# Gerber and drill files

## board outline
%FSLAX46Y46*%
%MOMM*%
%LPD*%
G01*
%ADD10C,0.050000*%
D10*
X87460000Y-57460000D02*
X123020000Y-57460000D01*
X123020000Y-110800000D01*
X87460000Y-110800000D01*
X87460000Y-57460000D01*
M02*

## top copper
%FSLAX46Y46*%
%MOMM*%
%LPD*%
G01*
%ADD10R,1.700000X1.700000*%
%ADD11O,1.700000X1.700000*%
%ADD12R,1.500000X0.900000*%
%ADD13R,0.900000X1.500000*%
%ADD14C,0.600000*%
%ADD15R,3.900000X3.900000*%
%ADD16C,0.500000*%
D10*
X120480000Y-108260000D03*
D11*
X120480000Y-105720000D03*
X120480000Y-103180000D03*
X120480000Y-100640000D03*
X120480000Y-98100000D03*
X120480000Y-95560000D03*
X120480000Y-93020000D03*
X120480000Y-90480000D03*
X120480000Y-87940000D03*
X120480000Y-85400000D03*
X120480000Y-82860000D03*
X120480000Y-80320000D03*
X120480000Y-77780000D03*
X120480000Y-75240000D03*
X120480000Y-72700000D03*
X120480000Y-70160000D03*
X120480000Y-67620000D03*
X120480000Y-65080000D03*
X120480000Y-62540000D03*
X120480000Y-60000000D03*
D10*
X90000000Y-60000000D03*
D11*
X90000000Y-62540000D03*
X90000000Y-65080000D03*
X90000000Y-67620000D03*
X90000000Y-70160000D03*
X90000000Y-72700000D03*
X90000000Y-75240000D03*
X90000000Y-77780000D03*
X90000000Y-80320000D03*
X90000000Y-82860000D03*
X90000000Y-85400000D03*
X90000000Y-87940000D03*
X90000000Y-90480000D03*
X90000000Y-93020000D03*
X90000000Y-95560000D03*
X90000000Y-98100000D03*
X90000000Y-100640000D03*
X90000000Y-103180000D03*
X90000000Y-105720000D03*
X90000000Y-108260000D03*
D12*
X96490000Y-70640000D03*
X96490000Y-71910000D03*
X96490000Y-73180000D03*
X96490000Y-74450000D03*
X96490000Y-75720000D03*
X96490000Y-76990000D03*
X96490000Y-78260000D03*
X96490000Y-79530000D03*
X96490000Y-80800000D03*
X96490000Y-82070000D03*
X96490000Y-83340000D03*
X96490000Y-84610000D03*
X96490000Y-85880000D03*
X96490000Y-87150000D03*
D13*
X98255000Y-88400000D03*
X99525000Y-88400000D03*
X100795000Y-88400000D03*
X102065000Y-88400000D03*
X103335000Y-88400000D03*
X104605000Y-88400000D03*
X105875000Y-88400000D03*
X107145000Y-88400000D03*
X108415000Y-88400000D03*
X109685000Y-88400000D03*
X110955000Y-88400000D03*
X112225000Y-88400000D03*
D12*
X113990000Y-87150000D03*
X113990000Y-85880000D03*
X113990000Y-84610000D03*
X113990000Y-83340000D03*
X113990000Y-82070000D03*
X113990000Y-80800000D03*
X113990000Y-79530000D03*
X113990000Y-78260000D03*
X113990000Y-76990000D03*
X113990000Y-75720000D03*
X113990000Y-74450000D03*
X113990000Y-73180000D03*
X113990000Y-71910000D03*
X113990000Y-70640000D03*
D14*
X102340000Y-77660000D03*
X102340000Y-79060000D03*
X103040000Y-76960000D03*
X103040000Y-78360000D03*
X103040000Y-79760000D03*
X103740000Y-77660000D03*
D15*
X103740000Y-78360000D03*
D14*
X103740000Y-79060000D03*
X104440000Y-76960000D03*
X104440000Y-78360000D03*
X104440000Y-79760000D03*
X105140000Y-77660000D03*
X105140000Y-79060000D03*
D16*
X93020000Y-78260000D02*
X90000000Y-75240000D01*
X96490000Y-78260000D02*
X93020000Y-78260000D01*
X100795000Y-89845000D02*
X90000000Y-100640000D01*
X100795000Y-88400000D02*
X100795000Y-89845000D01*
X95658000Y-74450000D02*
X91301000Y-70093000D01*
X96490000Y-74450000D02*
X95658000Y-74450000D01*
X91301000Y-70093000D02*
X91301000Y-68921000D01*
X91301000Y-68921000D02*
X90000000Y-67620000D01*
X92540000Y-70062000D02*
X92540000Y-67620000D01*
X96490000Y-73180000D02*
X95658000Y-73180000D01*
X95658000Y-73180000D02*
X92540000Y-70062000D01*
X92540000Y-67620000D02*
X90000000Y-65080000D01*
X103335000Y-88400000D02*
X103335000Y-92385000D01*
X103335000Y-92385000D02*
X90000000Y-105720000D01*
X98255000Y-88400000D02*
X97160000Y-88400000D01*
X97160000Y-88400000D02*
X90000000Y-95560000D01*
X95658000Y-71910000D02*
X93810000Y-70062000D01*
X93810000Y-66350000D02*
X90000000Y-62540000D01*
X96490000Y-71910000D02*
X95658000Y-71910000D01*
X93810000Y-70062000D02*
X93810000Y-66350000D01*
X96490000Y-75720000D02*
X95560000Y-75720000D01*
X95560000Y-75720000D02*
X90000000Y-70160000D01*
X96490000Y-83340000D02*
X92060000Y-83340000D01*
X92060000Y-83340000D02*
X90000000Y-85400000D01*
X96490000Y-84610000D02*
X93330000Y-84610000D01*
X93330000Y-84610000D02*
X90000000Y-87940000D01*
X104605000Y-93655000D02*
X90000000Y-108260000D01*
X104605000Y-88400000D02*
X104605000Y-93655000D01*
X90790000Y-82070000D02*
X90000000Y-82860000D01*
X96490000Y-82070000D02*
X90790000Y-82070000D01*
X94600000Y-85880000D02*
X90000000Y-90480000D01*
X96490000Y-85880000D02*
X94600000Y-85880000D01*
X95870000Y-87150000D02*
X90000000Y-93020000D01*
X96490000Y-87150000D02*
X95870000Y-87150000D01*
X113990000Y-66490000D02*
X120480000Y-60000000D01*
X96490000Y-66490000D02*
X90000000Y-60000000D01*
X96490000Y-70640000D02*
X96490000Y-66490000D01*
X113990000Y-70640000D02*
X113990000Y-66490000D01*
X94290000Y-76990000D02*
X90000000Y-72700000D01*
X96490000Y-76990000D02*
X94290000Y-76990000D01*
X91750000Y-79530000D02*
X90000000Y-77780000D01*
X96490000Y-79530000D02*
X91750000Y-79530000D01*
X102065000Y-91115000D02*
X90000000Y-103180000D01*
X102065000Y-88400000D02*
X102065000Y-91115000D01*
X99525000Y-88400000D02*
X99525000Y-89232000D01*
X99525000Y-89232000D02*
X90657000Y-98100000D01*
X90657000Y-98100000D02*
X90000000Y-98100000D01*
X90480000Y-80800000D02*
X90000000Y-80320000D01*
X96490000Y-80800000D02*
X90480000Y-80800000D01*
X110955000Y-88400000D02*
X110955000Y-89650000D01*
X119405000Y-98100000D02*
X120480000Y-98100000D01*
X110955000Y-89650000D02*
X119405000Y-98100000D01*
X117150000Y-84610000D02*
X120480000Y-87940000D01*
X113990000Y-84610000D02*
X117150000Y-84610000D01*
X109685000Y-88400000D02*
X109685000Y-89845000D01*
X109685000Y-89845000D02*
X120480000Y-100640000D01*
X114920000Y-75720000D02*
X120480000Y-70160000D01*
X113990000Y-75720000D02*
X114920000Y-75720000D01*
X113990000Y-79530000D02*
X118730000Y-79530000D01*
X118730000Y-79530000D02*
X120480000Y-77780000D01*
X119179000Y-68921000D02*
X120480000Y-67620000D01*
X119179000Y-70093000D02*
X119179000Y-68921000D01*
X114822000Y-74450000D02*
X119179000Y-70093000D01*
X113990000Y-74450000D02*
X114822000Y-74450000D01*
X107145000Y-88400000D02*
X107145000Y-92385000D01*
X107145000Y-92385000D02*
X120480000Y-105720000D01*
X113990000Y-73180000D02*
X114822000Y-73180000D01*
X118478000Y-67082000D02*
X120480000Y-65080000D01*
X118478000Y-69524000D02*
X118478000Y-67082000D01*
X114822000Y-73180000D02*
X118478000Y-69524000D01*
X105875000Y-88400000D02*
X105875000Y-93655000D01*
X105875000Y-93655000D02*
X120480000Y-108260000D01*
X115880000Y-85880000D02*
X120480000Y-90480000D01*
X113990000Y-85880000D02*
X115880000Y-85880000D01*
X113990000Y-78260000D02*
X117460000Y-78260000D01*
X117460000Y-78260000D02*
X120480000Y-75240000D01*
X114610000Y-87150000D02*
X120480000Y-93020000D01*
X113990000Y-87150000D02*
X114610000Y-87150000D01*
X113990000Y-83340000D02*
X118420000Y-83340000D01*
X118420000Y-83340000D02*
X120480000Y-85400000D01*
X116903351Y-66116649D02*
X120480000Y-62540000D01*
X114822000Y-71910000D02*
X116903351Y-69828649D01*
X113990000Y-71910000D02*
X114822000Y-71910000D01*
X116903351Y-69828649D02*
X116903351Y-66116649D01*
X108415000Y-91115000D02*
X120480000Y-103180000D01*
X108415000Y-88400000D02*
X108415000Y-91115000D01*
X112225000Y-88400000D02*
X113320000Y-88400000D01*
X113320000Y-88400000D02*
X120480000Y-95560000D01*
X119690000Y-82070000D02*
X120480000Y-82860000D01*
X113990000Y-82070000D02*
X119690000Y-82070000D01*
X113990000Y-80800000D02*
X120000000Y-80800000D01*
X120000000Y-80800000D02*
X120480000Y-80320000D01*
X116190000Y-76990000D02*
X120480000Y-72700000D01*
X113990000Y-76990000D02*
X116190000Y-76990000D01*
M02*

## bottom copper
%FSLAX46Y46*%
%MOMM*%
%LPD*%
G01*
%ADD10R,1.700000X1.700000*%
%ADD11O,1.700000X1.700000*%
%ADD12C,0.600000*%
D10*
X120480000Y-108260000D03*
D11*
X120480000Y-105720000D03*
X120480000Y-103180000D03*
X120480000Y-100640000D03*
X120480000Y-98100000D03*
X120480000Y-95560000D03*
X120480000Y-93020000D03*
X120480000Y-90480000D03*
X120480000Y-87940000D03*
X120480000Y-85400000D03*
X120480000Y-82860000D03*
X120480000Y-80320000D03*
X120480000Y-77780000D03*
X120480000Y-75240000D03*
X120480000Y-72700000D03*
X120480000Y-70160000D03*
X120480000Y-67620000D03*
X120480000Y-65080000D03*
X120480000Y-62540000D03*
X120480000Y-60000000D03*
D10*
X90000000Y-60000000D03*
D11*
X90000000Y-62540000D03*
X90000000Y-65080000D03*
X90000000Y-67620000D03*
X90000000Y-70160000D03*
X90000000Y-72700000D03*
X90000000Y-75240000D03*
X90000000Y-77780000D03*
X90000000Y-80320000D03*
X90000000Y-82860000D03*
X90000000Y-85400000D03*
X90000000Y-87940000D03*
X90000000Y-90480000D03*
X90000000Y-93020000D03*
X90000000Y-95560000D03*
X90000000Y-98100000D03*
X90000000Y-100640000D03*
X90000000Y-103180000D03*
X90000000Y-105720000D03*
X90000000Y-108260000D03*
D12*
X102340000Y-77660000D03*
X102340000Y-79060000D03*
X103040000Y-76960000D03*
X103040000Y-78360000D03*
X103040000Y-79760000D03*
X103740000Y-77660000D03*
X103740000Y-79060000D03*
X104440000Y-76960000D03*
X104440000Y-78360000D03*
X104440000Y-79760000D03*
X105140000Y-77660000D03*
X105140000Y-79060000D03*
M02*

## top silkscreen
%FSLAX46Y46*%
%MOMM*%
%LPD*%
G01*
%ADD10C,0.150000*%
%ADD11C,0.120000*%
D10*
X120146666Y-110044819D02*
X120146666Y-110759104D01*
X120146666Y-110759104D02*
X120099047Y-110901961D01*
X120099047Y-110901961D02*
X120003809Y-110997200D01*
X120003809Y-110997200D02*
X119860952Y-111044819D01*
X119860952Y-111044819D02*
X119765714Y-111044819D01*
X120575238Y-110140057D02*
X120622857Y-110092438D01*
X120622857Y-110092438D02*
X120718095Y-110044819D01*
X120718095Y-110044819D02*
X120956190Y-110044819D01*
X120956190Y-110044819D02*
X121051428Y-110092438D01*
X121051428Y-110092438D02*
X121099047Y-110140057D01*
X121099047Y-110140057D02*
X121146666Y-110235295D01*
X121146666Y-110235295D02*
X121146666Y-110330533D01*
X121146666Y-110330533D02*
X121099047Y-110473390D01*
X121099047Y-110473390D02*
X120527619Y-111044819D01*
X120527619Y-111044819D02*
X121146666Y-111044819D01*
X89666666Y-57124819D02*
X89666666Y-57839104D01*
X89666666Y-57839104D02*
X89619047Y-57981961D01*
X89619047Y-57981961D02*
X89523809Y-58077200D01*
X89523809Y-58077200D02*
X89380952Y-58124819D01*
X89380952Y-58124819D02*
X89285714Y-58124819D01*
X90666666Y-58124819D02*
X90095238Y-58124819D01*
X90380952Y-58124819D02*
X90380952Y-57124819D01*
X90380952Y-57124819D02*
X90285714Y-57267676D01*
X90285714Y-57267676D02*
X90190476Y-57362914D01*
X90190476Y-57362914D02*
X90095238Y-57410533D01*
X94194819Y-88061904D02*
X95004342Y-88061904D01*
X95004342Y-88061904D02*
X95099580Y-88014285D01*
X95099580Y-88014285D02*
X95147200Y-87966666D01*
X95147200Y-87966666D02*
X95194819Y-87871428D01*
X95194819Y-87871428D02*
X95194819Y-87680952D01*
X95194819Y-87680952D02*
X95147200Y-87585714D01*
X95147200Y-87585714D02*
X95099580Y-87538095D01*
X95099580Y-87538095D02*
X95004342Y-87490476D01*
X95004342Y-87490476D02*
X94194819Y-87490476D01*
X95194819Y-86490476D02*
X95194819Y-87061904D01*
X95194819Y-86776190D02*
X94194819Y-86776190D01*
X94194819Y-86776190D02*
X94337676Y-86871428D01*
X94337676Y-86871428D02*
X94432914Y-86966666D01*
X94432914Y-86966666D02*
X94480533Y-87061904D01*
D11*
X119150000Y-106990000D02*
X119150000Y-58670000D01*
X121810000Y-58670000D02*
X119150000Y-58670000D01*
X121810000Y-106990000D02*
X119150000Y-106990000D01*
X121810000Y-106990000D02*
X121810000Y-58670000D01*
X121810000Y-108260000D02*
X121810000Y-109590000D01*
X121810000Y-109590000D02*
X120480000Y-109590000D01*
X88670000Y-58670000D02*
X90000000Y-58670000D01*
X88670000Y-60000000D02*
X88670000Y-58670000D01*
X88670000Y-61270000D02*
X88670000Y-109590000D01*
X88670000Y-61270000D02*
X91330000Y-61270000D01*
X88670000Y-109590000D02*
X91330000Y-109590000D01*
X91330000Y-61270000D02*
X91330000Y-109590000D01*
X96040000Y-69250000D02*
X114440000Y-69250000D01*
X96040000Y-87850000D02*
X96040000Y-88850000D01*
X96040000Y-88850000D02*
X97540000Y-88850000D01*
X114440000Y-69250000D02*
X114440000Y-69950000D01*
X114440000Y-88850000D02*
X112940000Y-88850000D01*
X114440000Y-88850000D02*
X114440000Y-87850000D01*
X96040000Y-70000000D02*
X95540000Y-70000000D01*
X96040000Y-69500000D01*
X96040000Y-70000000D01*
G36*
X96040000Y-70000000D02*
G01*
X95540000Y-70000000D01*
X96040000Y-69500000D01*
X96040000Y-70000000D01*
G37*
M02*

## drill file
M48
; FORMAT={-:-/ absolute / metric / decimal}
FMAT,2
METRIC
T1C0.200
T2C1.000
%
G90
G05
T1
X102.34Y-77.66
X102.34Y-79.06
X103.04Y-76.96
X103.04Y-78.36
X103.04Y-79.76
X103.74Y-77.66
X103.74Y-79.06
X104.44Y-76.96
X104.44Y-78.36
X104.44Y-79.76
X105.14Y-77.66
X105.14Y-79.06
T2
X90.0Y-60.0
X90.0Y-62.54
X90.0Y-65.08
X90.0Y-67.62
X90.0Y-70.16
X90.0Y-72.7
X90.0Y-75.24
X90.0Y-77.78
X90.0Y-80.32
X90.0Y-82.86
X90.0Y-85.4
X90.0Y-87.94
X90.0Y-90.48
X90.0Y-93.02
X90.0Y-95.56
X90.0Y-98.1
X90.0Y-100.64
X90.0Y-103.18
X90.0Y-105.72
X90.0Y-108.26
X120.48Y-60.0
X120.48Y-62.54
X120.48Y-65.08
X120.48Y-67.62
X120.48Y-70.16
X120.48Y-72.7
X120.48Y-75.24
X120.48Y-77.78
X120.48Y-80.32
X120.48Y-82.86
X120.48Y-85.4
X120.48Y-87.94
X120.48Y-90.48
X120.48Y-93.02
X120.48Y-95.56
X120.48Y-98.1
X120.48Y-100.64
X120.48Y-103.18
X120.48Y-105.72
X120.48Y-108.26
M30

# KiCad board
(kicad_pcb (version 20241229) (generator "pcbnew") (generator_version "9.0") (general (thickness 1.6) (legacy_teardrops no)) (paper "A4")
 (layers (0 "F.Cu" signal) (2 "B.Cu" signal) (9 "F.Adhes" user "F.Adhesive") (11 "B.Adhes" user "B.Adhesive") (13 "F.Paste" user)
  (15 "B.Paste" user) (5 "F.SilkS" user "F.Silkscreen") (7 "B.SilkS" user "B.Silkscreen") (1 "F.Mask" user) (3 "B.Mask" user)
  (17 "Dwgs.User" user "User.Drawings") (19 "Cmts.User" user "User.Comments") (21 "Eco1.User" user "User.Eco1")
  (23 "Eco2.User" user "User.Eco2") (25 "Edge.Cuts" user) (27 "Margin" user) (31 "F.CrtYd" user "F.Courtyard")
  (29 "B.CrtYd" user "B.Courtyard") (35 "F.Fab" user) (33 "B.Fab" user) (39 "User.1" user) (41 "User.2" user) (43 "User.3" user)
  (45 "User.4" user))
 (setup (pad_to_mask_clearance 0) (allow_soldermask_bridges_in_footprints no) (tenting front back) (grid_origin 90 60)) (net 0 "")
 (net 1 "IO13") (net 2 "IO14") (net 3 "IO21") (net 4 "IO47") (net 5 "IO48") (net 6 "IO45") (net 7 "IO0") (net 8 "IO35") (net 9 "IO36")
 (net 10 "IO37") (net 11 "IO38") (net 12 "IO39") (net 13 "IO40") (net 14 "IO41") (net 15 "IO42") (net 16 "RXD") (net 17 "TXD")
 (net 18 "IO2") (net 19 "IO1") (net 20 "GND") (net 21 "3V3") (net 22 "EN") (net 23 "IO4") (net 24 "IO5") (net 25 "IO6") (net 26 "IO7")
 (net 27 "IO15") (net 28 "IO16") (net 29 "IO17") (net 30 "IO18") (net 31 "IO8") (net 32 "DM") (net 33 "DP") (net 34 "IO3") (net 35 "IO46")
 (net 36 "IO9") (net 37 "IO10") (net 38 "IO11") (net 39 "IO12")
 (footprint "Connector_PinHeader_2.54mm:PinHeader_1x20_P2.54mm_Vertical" (layer "F.Cu") (at 120.48 108.26 180)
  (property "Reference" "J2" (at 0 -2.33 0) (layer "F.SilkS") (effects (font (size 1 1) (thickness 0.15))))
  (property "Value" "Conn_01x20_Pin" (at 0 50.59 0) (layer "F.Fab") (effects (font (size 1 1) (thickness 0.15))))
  (fp_line (start 1.33 1.27) (end 1.33 49.59) (stroke (width 0.12) (type solid)) (layer "F.SilkS"))
  (fp_line (start -1.33 49.59) (end 1.33 49.59) (stroke (width 0.12) (type solid)) (layer "F.SilkS"))
  (fp_line (start -1.33 1.27) (end 1.33 1.27) (stroke (width 0.12) (type solid)) (layer "F.SilkS"))
  (fp_line (start -1.33 1.27) (end -1.33 49.59) (stroke (width 0.12) (type solid)) (layer "F.SilkS"))
  (fp_line (start -1.33 0) (end -1.33 -1.33) (stroke (width 0.12) (type solid)) (layer "F.SilkS"))
  (fp_line (start -1.33 -1.33) (end 0 -1.33) (stroke (width 0.12) (type solid)) (layer "F.SilkS"))
  (pad "1" thru_hole rect (at 0 0 180) (size 1.7 1.7) (drill 1) (layers "*.Cu" "*.Mask") (remove_unused_layers no) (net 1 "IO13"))
  (pad "2" thru_hole oval (at 0 2.54 180) (size 1.7 1.7) (drill 1) (layers "*.Cu" "*.Mask") (remove_unused_layers no) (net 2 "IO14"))
  (pad "3" thru_hole oval (at 0 5.08 180) (size 1.7 1.7) (drill 1) (layers "*.Cu" "*.Mask") (remove_unused_layers no) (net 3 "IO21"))
  (pad "4" thru_hole oval (at 0 7.62 180) (size 1.7 1.7) (drill 1) (layers "*.Cu" "*.Mask") (remove_unused_layers no) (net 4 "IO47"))
  (pad "5" thru_hole oval (at 0 10.16 180) (size 1.7 1.7) (drill 1) (layers "*.Cu" "*.Mask") (remove_unused_layers no) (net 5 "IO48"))
  (pad "6" thru_hole oval (at 0 12.7 180) (size 1.7 1.7) (drill 1) (layers "*.Cu" "*.Mask") (remove_unused_layers no) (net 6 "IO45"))
  (pad "7" thru_hole oval (at 0 15.24 180) (size 1.7 1.7) (drill 1) (layers "*.Cu" "*.Mask") (remove_unused_layers no) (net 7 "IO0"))
  (pad "8" thru_hole oval (at 0 17.78 180) (size 1.7 1.7) (drill 1) (layers "*.Cu" "*.Mask") (remove_unused_layers no) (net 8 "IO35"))
  (pad "9" thru_hole oval (at 0 20.32 180) (size 1.7 1.7) (drill 1) (layers "*.Cu" "*.Mask") (remove_unused_layers no) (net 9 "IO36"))
  (pad "10" thru_hole oval (at 0 22.86 180) (size 1.7 1.7) (drill 1) (layers "*.Cu" "*.Mask") (remove_unused_layers no) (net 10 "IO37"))
  (pad "11" thru_hole oval (at 0 25.4 180) (size 1.7 1.7) (drill 1) (layers "*.Cu" "*.Mask") (remove_unused_layers no) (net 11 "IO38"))
  (pad "12" thru_hole oval (at 0 27.94 180) (size 1.7 1.7) (drill 1) (layers "*.Cu" "*.Mask") (remove_unused_layers no) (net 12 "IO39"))
  (pad "13" thru_hole oval (at 0 30.48 180) (size 1.7 1.7) (drill 1) (layers "*.Cu" "*.Mask") (remove_unused_layers no) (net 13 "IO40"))
  (pad "14" thru_hole oval (at 0 33.02 180) (size 1.7 1.7) (drill 1) (layers "*.Cu" "*.Mask") (remove_unused_layers no) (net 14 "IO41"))
  (pad "15" thru_hole oval (at 0 35.56 180) (size 1.7 1.7) (drill 1) (layers "*.Cu" "*.Mask") (remove_unused_layers no) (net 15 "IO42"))
  (pad "16" thru_hole oval (at 0 38.1 180) (size 1.7 1.7) (drill 1) (layers "*.Cu" "*.Mask") (remove_unused_layers no) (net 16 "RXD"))
  (pad "17" thru_hole oval (at 0 40.64 180) (size 1.7 1.7) (drill 1) (layers "*.Cu" "*.Mask") (remove_unused_layers no) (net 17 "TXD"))
  (pad "18" thru_hole oval (at 0 43.18 180) (size 1.7 1.7) (drill 1) (layers "*.Cu" "*.Mask") (remove_unused_layers no) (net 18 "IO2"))
  (pad "19" thru_hole oval (at 0 45.72 180) (size 1.7 1.7) (drill 1) (layers "*.Cu" "*.Mask") (remove_unused_layers no) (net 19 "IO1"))
  (pad "20" thru_hole oval (at 0 48.26 180) (size 1.7 1.7) (drill 1) (layers "*.Cu" "*.Mask") (remove_unused_layers no) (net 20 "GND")))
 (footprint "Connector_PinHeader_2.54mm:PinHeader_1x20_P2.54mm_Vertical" (layer "F.Cu") (at 90 60)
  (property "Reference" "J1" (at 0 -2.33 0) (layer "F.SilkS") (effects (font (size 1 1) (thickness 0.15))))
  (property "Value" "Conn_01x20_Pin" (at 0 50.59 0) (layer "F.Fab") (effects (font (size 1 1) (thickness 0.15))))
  (fp_line (start -1.33 -1.33) (end 0 -1.33) (stroke (width 0.12) (type solid)) (layer "F.SilkS"))
  (fp_line (start -1.33 0) (end -1.33 -1.33) (stroke (width 0.12) (type solid)) (layer "F.SilkS"))
  (fp_line (start -1.33 1.27) (end -1.33 49.59) (stroke (width 0.12) (type solid)) (layer "F.SilkS"))
  (fp_line (start -1.33 1.27) (end 1.33 1.27) (stroke (width 0.12) (type solid)) (layer "F.SilkS"))
  (fp_line (start -1.33 49.59) (end 1.33 49.59) (stroke (width 0.12) (type solid)) (layer "F.SilkS"))
  (fp_line (start 1.33 1.27) (end 1.33 49.59) (stroke (width 0.12) (type solid)) (layer "F.SilkS"))
  (pad "1" thru_hole rect (at 0 0) (size 1.7 1.7) (drill 1) (layers "*.Cu" "*.Mask") (remove_unused_layers no) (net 20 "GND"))
  (pad "2" thru_hole oval (at 0 2.54) (size 1.7 1.7) (drill 1) (layers "*.Cu" "*.Mask") (remove_unused_layers no) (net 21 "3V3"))
  (pad "3" thru_hole oval (at 0 5.08) (size 1.7 1.7) (drill 1) (layers "*.Cu" "*.Mask") (remove_unused_layers no) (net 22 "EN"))
  (pad "4" thru_hole oval (at 0 7.62) (size 1.7 1.7) (drill 1) (layers "*.Cu" "*.Mask") (remove_unused_layers no) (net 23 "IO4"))
  (pad "5" thru_hole oval (at 0 10.16) (size 1.7 1.7) (drill 1) (layers "*.Cu" "*.Mask") (remove_unused_layers no) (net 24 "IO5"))
  (pad "6" thru_hole oval (at 0 12.7) (size 1.7 1.7) (drill 1) (layers "*.Cu" "*.Mask") (remove_unused_layers no) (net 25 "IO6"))
  (pad "7" thru_hole oval (at 0 15.24) (size 1.7 1.7) (drill 1) (layers "*.Cu" "*.Mask") (remove_unused_layers no) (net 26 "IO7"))
  (pad "8" thru_hole oval (at 0 17.78) (size 1.7 1.7) (drill 1) (layers "*.Cu" "*.Mask") (remove_unused_layers no) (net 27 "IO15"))
  (pad "9" thru_hole oval (at 0 20.32) (size 1.7 1.7) (drill 1) (layers "*.Cu" "*.Mask") (remove_unused_layers no) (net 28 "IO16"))
  (pad "10" thru_hole oval (at 0 22.86) (size 1.7 1.7) (drill 1) (layers "*.Cu" "*.Mask") (remove_unused_layers no) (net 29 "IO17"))
  (pad "11" thru_hole oval (at 0 25.4) (size 1.7 1.7) (drill 1) (layers "*.Cu" "*.Mask") (remove_unused_layers no) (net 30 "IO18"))
  (pad "12" thru_hole oval (at 0 27.94) (size 1.7 1.7) (drill 1) (layers "*.Cu" "*.Mask") (remove_unused_layers no) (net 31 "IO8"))
  (pad "13" thru_hole oval (at 0 30.48) (size 1.7 1.7) (drill 1) (layers "*.Cu" "*.Mask") (remove_unused_layers no) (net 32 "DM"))
  (pad "14" thru_hole oval (at 0 33.02) (size 1.7 1.7) (drill 1) (layers "*.Cu" "*.Mask") (remove_unused_layers no) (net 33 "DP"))
  (pad "15" thru_hole oval (at 0 35.56) (size 1.7 1.7) (drill 1) (layers "*.Cu" "*.Mask") (remove_unused_layers no) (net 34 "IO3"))
  (pad "16" thru_hole oval (at 0 38.1) (size 1.7 1.7) (drill 1) (layers "*.Cu" "*.Mask") (remove_unused_layers no) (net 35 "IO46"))
  (pad "17" thru_hole oval (at 0 40.64) (size 1.7 1.7) (drill 1) (layers "*.Cu" "*.Mask") (remove_unused_layers no) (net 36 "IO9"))
  (pad "18" thru_hole oval (at 0 43.18) (size 1.7 1.7) (drill 1) (layers "*.Cu" "*.Mask") (remove_unused_layers no) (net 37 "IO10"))
  (pad "19" thru_hole oval (at 0 45.72) (size 1.7 1.7) (drill 1) (layers "*.Cu" "*.Mask") (remove_unused_layers no) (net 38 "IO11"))
  (pad "20" thru_hole oval (at 0 48.26) (size 1.7 1.7) (drill 1) (layers "*.Cu" "*.Mask") (remove_unused_layers no) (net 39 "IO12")))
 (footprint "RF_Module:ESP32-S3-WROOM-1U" (layer "F.Cu") (at 105.24 79.05)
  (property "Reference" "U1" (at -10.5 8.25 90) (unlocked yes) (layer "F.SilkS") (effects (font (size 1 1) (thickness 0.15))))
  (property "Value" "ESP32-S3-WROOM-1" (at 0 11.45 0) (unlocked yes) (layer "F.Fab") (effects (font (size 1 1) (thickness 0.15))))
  (fp_line (start -9.2 -9.8) (end 9.2 -9.8) (stroke (width 0.12) (type solid)) (layer "F.SilkS"))
  (fp_line (start -9.2 8.8) (end -9.2 9.8) (stroke (width 0.12) (type solid)) (layer "F.SilkS"))
  (fp_line (start -9.2 9.8) (end -7.7 9.8) (stroke (width 0.12) (type solid)) (layer "F.SilkS"))
  (fp_line (start 9.2 -9.8) (end 9.2 -9.1) (stroke (width 0.12) (type solid)) (layer "F.SilkS"))
  (fp_line (start 9.2 9.8) (end 7.7 9.8) (stroke (width 0.12) (type solid)) (layer "F.SilkS"))
  (fp_line (start 9.2 9.8) (end 9.2 8.8) (stroke (width 0.12) (type solid)) (layer "F.SilkS"))
  (fp_poly
   (pts (xy -9.2 -9.05) (xy -9.7 -9.05) (xy -9.2 -9.55) (xy -9.2 -9.05)) (stroke (width 0.12) (type solid)) (fill yes) (layer "F.SilkS"))
  (pad "" smd rect (at -2.904394 0.71) (size 0.9 0.9) (layers "F.Paste"))
  (pad "" smd rect (at -2.9 -2.09) (size 0.9 0.9) (layers "F.Paste"))
  (pad "" smd rect (at -2.9 -0.69) (size 0.9 0.9) (layers "F.Paste"))
  (pad "" smd rect (at -1.504394 0.71) (size 0.9 0.9) (layers "F.Paste"))
  (pad "" smd rect (at -1.5 -2.09) (size 0.9 0.9) (layers "F.Paste"))
  (pad "" smd rect (at -1.5 -0.69) (size 0.9 0.9) (layers "F.Paste"))
  (pad "" smd rect (at -0.104394 0.71) (size 0.9 0.9) (layers "F.Paste"))
  (pad "" smd rect (at -0.1 -2.09) (size 0.9 0.9) (layers "F.Paste"))
  (pad "" smd rect (at -0.1 -0.69) (size 0.9 0.9) (layers "F.Paste"))
  (pad "1" smd rect (at -8.75 -8.41) (size 1.5 0.9) (layers "F.Cu" "F.Mask" "F.Paste") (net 20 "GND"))
  (pad "2" smd rect (at -8.75 -7.14) (size 1.5 0.9) (layers "F.Cu" "F.Mask" "F.Paste") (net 21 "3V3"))
  (pad "3" smd rect (at -8.75 -5.87) (size 1.5 0.9) (layers "F.Cu" "F.Mask" "F.Paste") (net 22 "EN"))
  (pad "4" smd rect (at -8.75 -4.6) (size 1.5 0.9) (layers "F.Cu" "F.Mask" "F.Paste") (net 23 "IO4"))
  (pad "5" smd rect (at -8.75 -3.33) (size 1.5 0.9) (layers "F.Cu" "F.Mask" "F.Paste") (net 24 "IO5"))
  (pad "6" smd rect (at -8.75 -2.06) (size 1.5 0.9) (layers "F.Cu" "F.Mask" "F.Paste") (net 25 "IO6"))
  (pad "7" smd rect (at -8.75 -0.79) (size 1.5 0.9) (layers "F.Cu" "F.Mask" "F.Paste") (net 26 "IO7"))
  (pad "8" smd rect (at -8.75 0.48) (size 1.5 0.9) (layers "F.Cu" "F.Mask" "F.Paste") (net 27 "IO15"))
  (pad "9" smd rect (at -8.75 1.75) (size 1.5 0.9) (layers "F.Cu" "F.Mask" "F.Paste") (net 28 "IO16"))
  (pad "10" smd rect (at -8.75 3.02) (size 1.5 0.9) (layers "F.Cu" "F.Mask" "F.Paste") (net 29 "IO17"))
  (pad "11" smd rect (at -8.75 4.29) (size 1.5 0.9) (layers "F.Cu" "F.Mask" "F.Paste") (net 30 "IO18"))
  (pad "12" smd rect (at -8.75 5.56) (size 1.5 0.9) (layers "F.Cu" "F.Mask" "F.Paste") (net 31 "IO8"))
  (pad "13" smd rect (at -8.75 6.83) (size 1.5 0.9) (layers "F.Cu" "F.Mask" "F.Paste") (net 32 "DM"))
  (pad "14" smd rect (at -8.75 8.1 180) (size 1.5 0.9) (layers "F.Cu" "F.Mask" "F.Paste") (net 33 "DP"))
  (pad "15" smd rect (at -6.985 9.35 270) (size 1.5 0.9) (layers "F.Cu" "F.Mask" "F.Paste") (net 34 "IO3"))
  (pad "16" smd rect (at -5.715 9.35 270) (size 1.5 0.9) (layers "F.Cu" "F.Mask" "F.Paste") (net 35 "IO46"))
  (pad "17" smd rect (at -4.445 9.35 270) (size 1.5 0.9) (layers "F.Cu" "F.Mask" "F.Paste") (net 36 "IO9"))
  (pad "18" smd rect (at -3.175 9.35 270) (size 1.5 0.9) (layers "F.Cu" "F.Mask" "F.Paste") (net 37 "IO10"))
  (pad "19" smd rect (at -1.905 9.35 270) (size 1.5 0.9) (layers "F.Cu" "F.Mask" "F.Paste") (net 38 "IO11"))
  (pad "20" smd rect (at -0.635 9.35 270) (size 1.5 0.9) (layers "F.Cu" "F.Mask" "F.Paste") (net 39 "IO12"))
  (pad "21" smd rect (at 0.635 9.35 270) (size 1.5 0.9) (layers "F.Cu" "F.Mask" "F.Paste") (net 1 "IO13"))
  (pad "22" smd rect (at 1.905 9.35 270) (size 1.5 0.9) (layers "F.Cu" "F.Mask" "F.Paste") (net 2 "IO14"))
  (pad "23" smd rect (at 3.175 9.35 270) (size 1.5 0.9) (layers "F.Cu" "F.Mask" "F.Paste") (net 3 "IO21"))
  (pad "24" smd rect (at 4.445 9.35 270) (size 1.5 0.9) (layers "F.Cu" "F.Mask" "F.Paste") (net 4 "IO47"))
  (pad "25" smd rect (at 5.715 9.35 270) (size 1.5 0.9) (layers "F.Cu" "F.Mask" "F.Paste") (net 5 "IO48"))
  (pad "26" smd rect (at 6.985 9.35 270) (size 1.5 0.9) (layers "F.Cu" "F.Mask" "F.Paste") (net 6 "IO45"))
  (pad "27" smd rect (at 8.75 8.1) (size 1.5 0.9) (layers "F.Cu" "F.Mask" "F.Paste") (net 7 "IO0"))
  (pad "28" smd rect (at 8.75 6.83) (size 1.5 0.9) (layers "F.Cu" "F.Mask" "F.Paste") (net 8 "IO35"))
  (pad "29" smd rect (at 8.75 5.56) (size 1.5 0.9) (layers "F.Cu" "F.Mask" "F.Paste") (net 9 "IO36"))
  (pad "30" smd rect (at 8.75 4.29) (size 1.5 0.9) (layers "F.Cu" "F.Mask" "F.Paste") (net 10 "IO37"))
  (pad "31" smd rect (at 8.75 3.02) (size 1.5 0.9) (layers "F.Cu" "F.Mask" "F.Paste") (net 11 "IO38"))
  (pad "32" smd rect (at 8.75 1.75) (size 1.5 0.9) (layers "F.Cu" "F.Mask" "F.Paste") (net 12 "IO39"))
  (pad "33" smd rect (at 8.75 0.48) (size 1.5 0.9) (layers "F.Cu" "F.Mask" "F.Paste") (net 13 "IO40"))
  (pad "34" smd rect (at 8.75 -0.79) (size 1.5 0.9) (layers "F.Cu" "F.Mask" "F.Paste") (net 14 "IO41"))
  (pad "35" smd rect (at 8.75 -2.06) (size 1.5 0.9) (layers "F.Cu" "F.Mask" "F.Paste") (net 15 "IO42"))
  (pad "36" smd rect (at 8.75 -3.33) (size 1.5 0.9) (layers "F.Cu" "F.Mask" "F.Paste") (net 16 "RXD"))
  (pad "37" smd rect (at 8.75 -4.6) (size 1.5 0.9) (layers "F.Cu" "F.Mask" "F.Paste") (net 17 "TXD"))
  (pad "38" smd rect (at 8.75 -5.87) (size 1.5 0.9) (layers "F.Cu" "F.Mask" "F.Paste") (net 18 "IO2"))
  (pad "39" smd rect (at 8.75 -7.14) (size 1.5 0.9) (layers "F.Cu" "F.Mask" "F.Paste") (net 19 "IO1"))
  (pad "40" smd rect (at 8.75 -8.41) (size 1.5 0.9) (layers "F.Cu" "F.Mask" "F.Paste") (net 20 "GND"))
  (pad "41" thru_hole circle (at -2.9 -1.39) (size 0.6 0.6) (drill 0.2) (layers "*.Cu" "F.Mask") (remove_unused_layers no) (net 20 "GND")
   (zone_connect 2))
  (pad "41" thru_hole circle (at -2.9 0.01) (size 0.6 0.6) (drill 0.2) (layers "*.Cu" "F.Mask") (remove_unused_layers no) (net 20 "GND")
   (zone_connect 2))
  (pad "41" thru_hole circle (at -2.2 -2.09) (size 0.6 0.6) (drill 0.2) (layers "*.Cu" "F.Mask") (remove_unused_layers no) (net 20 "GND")
   (zone_connect 2))
  (pad "41" thru_hole circle (at -2.2 -0.69) (size 0.6 0.6) (drill 0.2) (layers "*.Cu" "F.Mask") (remove_unused_layers no) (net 20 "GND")
   (zone_connect 2))
  (pad "41" thru_hole circle (at -2.2 0.71) (size 0.6 0.6) (drill 0.2) (layers "*.Cu" "F.Mask") (remove_unused_layers no) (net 20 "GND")
   (zone_connect 2))
  (pad "41" thru_hole circle (at -1.5 -1.39) (size 0.6 0.6) (drill 0.2) (layers "*.Cu" "F.Mask") (remove_unused_layers no) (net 20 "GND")
   (zone_connect 2))
  (pad "41" smd rect (at -1.5 -0.69) (size 3.9 3.9) (layers "F.Cu" "F.Mask") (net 20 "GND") (zone_connect 2))
  (pad "41" thru_hole circle (at -1.5 0.01) (size 0.6 0.6) (drill 0.2) (layers "*.Cu" "F.Mask") (remove_unused_layers no) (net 20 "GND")
   (zone_connect 2))
  (pad "41" thru_hole circle (at -0.8 -2.09) (size 0.6 0.6) (drill 0.2) (layers "*.Cu" "F.Mask") (remove_unused_layers no) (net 20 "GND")
   (zone_connect 2))
  (pad "41" thru_hole circle (at -0.8 -0.69) (size 0.6 0.6) (drill 0.2) (layers "*.Cu" "F.Mask") (remove_unused_layers no) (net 20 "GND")
   (zone_connect 2))
  (pad "41" thru_hole circle (at -0.8 0.71) (size 0.6 0.6) (drill 0.2) (layers "*.Cu" "F.Mask") (remove_unused_layers no) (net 20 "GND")
   (zone_connect 2))
  (pad "41" thru_hole circle (at -0.1 -1.39) (size 0.6 0.6) (drill 0.2) (layers "*.Cu" "F.Mask") (remove_unused_layers no) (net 20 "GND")
   (zone_connect 2))
  (pad "41" thru_hole circle (at -0.1 0.01) (size 0.6 0.6) (drill 0.2) (layers "*.Cu" "F.Mask") (remove_unused_layers no) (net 20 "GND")
   (zone_connect 2)))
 (gr_rect (start 87.46 57.46) (end 123.02 110.8) (stroke (width 0.05) (type default)) (fill no) (layer "Edge.Cuts"))
 (segment (start 93.02 78.26) (end 90 75.24) (width 0.5) (layer "F.Cu") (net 26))
 (segment (start 96.49 78.26) (end 93.02 78.26) (width 0.5) (layer "F.Cu") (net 26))
 (segment (start 100.795 89.845) (end 90 100.64) (width 0.5) (layer "F.Cu") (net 36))
 (segment (start 100.795 88.4) (end 100.795 89.845) (width 0.5) (layer "F.Cu") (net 36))
 (segment (start 95.658 74.45) (end 91.301 70.093) (width 0.5) (layer "F.Cu") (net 23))
 (segment (start 96.49 74.45) (end 95.658 74.45) (width 0.5) (layer "F.Cu") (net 23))
 (segment (start 91.301 70.093) (end 91.301 68.921) (width 0.5) (layer "F.Cu") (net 23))
 (segment (start 91.301 68.921) (end 90 67.62) (width 0.5) (layer "F.Cu") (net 23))
 (segment (start 92.54 70.062) (end 92.54 67.62) (width 0.5) (layer "F.Cu") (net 22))
 (segment (start 96.49 73.18) (end 95.658 73.18) (width 0.5) (layer "F.Cu") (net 22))
 (segment (start 95.658 73.18) (end 92.54 70.062) (width 0.5) (layer "F.Cu") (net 22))
 (segment (start 92.54 67.62) (end 90 65.08) (width 0.5) (layer "F.Cu") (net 22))
 (segment (start 103.335 88.4) (end 103.335 92.385) (width 0.5) (layer "F.Cu") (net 38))
 (segment (start 103.335 92.385) (end 90 105.72) (width 0.5) (layer "F.Cu") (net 38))
 (segment (start 98.255 88.4) (end 97.16 88.4) (width 0.5) (layer "F.Cu") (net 34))
 (segment (start 97.16 88.4) (end 90 95.56) (width 0.5) (layer "F.Cu") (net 34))
 (segment (start 95.658 71.91) (end 93.81 70.062) (width 0.5) (layer "F.Cu") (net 21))
 (segment (start 93.81 66.35) (end 90 62.54) (width 0.5) (layer "F.Cu") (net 21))
 (segment (start 96.49 71.91) (end 95.658 71.91) (width 0.5) (layer "F.Cu") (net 21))
 (segment (start 93.81 70.062) (end 93.81 66.35) (width 0.5) (layer "F.Cu") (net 21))
 (segment (start 96.49 75.72) (end 95.56 75.72) (width 0.5) (layer "F.Cu") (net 24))
 (segment (start 95.56 75.72) (end 90 70.16) (width 0.5) (layer "F.Cu") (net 24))
 (segment (start 96.49 83.34) (end 92.06 83.34) (width 0.5) (layer "F.Cu") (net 30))
 (segment (start 92.06 83.34) (end 90 85.4) (width 0.5) (layer "F.Cu") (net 30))
 (segment (start 96.49 84.61) (end 93.33 84.61) (width 0.5) (layer "F.Cu") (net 31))
 (segment (start 93.33 84.61) (end 90 87.94) (width 0.5) (layer "F.Cu") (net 31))
 (segment (start 104.605 93.655) (end 90 108.26) (width 0.5) (layer "F.Cu") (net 39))
 (segment (start 104.605 88.4) (end 104.605 93.655) (width 0.5) (layer "F.Cu") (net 39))
 (segment (start 90.79 82.07) (end 90 82.86) (width 0.5) (layer "F.Cu") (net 29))
 (segment (start 96.49 82.07) (end 90.79 82.07) (width 0.5) (layer "F.Cu") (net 29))
 (segment (start 94.6 85.88) (end 90 90.48) (width 0.5) (layer "F.Cu") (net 32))
 (segment (start 96.49 85.88) (end 94.6 85.88) (width 0.5) (layer "F.Cu") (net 32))
 (segment (start 95.87 87.15) (end 90 93.02) (width 0.5) (layer "F.Cu") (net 33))
 (segment (start 96.49 87.15) (end 95.87 87.15) (width 0.5) (layer "F.Cu") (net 33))
 (segment (start 113.99 66.49) (end 120.48 60) (width 0.5) (layer "F.Cu") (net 20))
 (segment (start 96.49 66.49) (end 90 60) (width 0.5) (layer "F.Cu") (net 20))
 (segment (start 96.49 70.64) (end 96.49 66.49) (width 0.5) (layer "F.Cu") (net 20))
 (segment (start 113.99 70.64) (end 113.99 66.49) (width 0.5) (layer "F.Cu") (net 20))
 (segment (start 94.29 76.99) (end 90 72.7) (width 0.5) (layer "F.Cu") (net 25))
 (segment (start 96.49 76.99) (end 94.29 76.99) (width 0.5) (layer "F.Cu") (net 25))
 (segment (start 91.75 79.53) (end 90 77.78) (width 0.5) (layer "F.Cu") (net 27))
 (segment (start 96.49 79.53) (end 91.75 79.53) (width 0.5) (layer "F.Cu") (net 27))
 (segment (start 102.065 91.115) (end 90 103.18) (width 0.5) (layer "F.Cu") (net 37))
 (segment (start 102.065 88.4) (end 102.065 91.115) (width 0.5) (layer "F.Cu") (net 37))
 (segment (start 99.525 88.4) (end 99.525 89.232) (width 0.5) (layer "F.Cu") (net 35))
 (segment (start 99.525 89.232) (end 90.657 98.1) (width 0.5) (layer "F.Cu") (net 35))
 (segment (start 90.657 98.1) (end 90 98.1) (width 0.5) (layer "F.Cu") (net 35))
 (segment (start 90.48 80.8) (end 90 80.32) (width 0.5) (layer "F.Cu") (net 28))
 (segment (start 96.49 80.8) (end 90.48 80.8) (width 0.5) (layer "F.Cu") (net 28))
 (segment (start 110.955 88.4) (end 110.955 89.65) (width 0.5) (layer "F.Cu") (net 5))
 (segment (start 119.405 98.1) (end 120.48 98.1) (width 0.5) (layer "F.Cu") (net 5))
 (segment (start 110.955 89.65) (end 119.405 98.1) (width 0.5) (layer "F.Cu") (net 5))
 (segment (start 117.15 84.61) (end 120.48 87.94) (width 0.5) (layer "F.Cu") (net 9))
 (segment (start 113.99 84.61) (end 117.15 84.61) (width 0.5) (layer "F.Cu") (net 9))
 (segment (start 109.685 88.4) (end 109.685 89.845) (width 0.5) (layer "F.Cu") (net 4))
 (segment (start 109.685 89.845) (end 120.48 100.64) (width 0.5) (layer "F.Cu") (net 4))
 (segment (start 114.92 75.72) (end 120.48 70.16) (width 0.5) (layer "F.Cu") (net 16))
 (segment (start 113.99 75.72) (end 114.92 75.72) (width 0.5) (layer "F.Cu") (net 16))
 (segment (start 113.99 79.53) (end 118.73 79.53) (width 0.5) (layer "F.Cu") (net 13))
 (segment (start 118.73 79.53) (end 120.48 77.78) (width 0.5) (layer "F.Cu") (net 13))
 (segment (start 119.179 68.921) (end 120.48 67.62) (width 0.5) (layer "F.Cu") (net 17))
 (segment (start 119.179 70.093) (end 119.179 68.921) (width 0.5) (layer "F.Cu") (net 17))
 (segment (start 114.822 74.45) (end 119.179 70.093) (width 0.5) (layer "F.Cu") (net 17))
 (segment (start 113.99 74.45) (end 114.822 74.45) (width 0.5) (layer "F.Cu") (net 17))
 (segment (start 107.145 88.4) (end 107.145 92.385) (width 0.5) (layer "F.Cu") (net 2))
 (segment (start 107.145 92.385) (end 120.48 105.72) (width 0.5) (layer "F.Cu") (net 2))
 (segment (start 113.99 73.18) (end 114.822 73.18) (width 0.5) (layer "F.Cu") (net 18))
 (segment (start 118.478 67.082) (end 120.48 65.08) (width 0.5) (layer "F.Cu") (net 18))
 (segment (start 118.478 69.524) (end 118.478 67.082) (width 0.5) (layer "F.Cu") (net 18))
 (segment (start 114.822 73.18) (end 118.478 69.524) (width 0.5) (layer "F.Cu") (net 18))
 (segment (start 105.875 88.4) (end 105.875 93.655) (width 0.5) (layer "F.Cu") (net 1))
 (segment (start 105.875 93.655) (end 120.48 108.26) (width 0.5) (layer "F.Cu") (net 1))
 (segment (start 115.88 85.88) (end 120.48 90.48) (width 0.5) (layer "F.Cu") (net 8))
 (segment (start 113.99 85.88) (end 115.88 85.88) (width 0.5) (layer "F.Cu") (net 8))
 (segment (start 113.99 78.26) (end 117.46 78.26) (width 0.5) (layer "F.Cu") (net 14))
 (segment (start 117.46 78.26) (end 120.48 75.24) (width 0.5) (layer "F.Cu") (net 14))
 (segment (start 114.61 87.15) (end 120.48 93.02) (width 0.5) (layer "F.Cu") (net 7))
 (segment (start 113.99 87.15) (end 114.61 87.15) (width 0.5) (layer "F.Cu") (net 7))
 (segment (start 113.99 83.34) (end 118.42 83.34) (width 0.5) (layer "F.Cu") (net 10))
 (segment (start 118.42 83.34) (end 120.48 85.4) (width 0.5) (layer "F.Cu") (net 10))
 (segment (start 116.903351 66.116649) (end 120.48 62.54) (width 0.5) (layer "F.Cu") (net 19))
 (segment (start 114.822 71.91) (end 116.903351 69.828649) (width 0.5) (layer "F.Cu") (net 19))
 (segment (start 113.99 71.91) (end 114.822 71.91) (width 0.5) (layer "F.Cu") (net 19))
 (segment (start 116.903351 69.828649) (end 116.903351 66.116649) (width 0.5) (layer "F.Cu") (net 19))
 (segment (start 108.415 91.115) (end 120.48 103.18) (width 0.5) (layer "F.Cu") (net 3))
 (segment (start 108.415 88.4) (end 108.415 91.115) (width 0.5) (layer "F.Cu") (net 3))
 (segment (start 112.225 88.4) (end 113.32 88.4) (width 0.5) (layer "F.Cu") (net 6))
 (segment (start 113.32 88.4) (end 120.48 95.56) (width 0.5) (layer "F.Cu") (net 6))
 (segment (start 119.69 82.07) (end 120.48 82.86) (width 0.5) (layer "F.Cu") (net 11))
 (segment (start 113.99 82.07) (end 119.69 82.07) (width 0.5) (layer "F.Cu") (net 11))
 (segment (start 113.99 80.8) (end 120 80.8) (width 0.5) (layer "F.Cu") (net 12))
 (segment (start 120 80.8) (end 120.48 80.32) (width 0.5) (layer "F.Cu") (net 12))
 (segment (start 116.19 76.99) (end 120.48 72.7) (width 0.5) (layer "F.Cu") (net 15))
 (segment (start 113.99 76.99) (end 116.19 76.99) (width 0.5) (layer "F.Cu") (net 15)))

